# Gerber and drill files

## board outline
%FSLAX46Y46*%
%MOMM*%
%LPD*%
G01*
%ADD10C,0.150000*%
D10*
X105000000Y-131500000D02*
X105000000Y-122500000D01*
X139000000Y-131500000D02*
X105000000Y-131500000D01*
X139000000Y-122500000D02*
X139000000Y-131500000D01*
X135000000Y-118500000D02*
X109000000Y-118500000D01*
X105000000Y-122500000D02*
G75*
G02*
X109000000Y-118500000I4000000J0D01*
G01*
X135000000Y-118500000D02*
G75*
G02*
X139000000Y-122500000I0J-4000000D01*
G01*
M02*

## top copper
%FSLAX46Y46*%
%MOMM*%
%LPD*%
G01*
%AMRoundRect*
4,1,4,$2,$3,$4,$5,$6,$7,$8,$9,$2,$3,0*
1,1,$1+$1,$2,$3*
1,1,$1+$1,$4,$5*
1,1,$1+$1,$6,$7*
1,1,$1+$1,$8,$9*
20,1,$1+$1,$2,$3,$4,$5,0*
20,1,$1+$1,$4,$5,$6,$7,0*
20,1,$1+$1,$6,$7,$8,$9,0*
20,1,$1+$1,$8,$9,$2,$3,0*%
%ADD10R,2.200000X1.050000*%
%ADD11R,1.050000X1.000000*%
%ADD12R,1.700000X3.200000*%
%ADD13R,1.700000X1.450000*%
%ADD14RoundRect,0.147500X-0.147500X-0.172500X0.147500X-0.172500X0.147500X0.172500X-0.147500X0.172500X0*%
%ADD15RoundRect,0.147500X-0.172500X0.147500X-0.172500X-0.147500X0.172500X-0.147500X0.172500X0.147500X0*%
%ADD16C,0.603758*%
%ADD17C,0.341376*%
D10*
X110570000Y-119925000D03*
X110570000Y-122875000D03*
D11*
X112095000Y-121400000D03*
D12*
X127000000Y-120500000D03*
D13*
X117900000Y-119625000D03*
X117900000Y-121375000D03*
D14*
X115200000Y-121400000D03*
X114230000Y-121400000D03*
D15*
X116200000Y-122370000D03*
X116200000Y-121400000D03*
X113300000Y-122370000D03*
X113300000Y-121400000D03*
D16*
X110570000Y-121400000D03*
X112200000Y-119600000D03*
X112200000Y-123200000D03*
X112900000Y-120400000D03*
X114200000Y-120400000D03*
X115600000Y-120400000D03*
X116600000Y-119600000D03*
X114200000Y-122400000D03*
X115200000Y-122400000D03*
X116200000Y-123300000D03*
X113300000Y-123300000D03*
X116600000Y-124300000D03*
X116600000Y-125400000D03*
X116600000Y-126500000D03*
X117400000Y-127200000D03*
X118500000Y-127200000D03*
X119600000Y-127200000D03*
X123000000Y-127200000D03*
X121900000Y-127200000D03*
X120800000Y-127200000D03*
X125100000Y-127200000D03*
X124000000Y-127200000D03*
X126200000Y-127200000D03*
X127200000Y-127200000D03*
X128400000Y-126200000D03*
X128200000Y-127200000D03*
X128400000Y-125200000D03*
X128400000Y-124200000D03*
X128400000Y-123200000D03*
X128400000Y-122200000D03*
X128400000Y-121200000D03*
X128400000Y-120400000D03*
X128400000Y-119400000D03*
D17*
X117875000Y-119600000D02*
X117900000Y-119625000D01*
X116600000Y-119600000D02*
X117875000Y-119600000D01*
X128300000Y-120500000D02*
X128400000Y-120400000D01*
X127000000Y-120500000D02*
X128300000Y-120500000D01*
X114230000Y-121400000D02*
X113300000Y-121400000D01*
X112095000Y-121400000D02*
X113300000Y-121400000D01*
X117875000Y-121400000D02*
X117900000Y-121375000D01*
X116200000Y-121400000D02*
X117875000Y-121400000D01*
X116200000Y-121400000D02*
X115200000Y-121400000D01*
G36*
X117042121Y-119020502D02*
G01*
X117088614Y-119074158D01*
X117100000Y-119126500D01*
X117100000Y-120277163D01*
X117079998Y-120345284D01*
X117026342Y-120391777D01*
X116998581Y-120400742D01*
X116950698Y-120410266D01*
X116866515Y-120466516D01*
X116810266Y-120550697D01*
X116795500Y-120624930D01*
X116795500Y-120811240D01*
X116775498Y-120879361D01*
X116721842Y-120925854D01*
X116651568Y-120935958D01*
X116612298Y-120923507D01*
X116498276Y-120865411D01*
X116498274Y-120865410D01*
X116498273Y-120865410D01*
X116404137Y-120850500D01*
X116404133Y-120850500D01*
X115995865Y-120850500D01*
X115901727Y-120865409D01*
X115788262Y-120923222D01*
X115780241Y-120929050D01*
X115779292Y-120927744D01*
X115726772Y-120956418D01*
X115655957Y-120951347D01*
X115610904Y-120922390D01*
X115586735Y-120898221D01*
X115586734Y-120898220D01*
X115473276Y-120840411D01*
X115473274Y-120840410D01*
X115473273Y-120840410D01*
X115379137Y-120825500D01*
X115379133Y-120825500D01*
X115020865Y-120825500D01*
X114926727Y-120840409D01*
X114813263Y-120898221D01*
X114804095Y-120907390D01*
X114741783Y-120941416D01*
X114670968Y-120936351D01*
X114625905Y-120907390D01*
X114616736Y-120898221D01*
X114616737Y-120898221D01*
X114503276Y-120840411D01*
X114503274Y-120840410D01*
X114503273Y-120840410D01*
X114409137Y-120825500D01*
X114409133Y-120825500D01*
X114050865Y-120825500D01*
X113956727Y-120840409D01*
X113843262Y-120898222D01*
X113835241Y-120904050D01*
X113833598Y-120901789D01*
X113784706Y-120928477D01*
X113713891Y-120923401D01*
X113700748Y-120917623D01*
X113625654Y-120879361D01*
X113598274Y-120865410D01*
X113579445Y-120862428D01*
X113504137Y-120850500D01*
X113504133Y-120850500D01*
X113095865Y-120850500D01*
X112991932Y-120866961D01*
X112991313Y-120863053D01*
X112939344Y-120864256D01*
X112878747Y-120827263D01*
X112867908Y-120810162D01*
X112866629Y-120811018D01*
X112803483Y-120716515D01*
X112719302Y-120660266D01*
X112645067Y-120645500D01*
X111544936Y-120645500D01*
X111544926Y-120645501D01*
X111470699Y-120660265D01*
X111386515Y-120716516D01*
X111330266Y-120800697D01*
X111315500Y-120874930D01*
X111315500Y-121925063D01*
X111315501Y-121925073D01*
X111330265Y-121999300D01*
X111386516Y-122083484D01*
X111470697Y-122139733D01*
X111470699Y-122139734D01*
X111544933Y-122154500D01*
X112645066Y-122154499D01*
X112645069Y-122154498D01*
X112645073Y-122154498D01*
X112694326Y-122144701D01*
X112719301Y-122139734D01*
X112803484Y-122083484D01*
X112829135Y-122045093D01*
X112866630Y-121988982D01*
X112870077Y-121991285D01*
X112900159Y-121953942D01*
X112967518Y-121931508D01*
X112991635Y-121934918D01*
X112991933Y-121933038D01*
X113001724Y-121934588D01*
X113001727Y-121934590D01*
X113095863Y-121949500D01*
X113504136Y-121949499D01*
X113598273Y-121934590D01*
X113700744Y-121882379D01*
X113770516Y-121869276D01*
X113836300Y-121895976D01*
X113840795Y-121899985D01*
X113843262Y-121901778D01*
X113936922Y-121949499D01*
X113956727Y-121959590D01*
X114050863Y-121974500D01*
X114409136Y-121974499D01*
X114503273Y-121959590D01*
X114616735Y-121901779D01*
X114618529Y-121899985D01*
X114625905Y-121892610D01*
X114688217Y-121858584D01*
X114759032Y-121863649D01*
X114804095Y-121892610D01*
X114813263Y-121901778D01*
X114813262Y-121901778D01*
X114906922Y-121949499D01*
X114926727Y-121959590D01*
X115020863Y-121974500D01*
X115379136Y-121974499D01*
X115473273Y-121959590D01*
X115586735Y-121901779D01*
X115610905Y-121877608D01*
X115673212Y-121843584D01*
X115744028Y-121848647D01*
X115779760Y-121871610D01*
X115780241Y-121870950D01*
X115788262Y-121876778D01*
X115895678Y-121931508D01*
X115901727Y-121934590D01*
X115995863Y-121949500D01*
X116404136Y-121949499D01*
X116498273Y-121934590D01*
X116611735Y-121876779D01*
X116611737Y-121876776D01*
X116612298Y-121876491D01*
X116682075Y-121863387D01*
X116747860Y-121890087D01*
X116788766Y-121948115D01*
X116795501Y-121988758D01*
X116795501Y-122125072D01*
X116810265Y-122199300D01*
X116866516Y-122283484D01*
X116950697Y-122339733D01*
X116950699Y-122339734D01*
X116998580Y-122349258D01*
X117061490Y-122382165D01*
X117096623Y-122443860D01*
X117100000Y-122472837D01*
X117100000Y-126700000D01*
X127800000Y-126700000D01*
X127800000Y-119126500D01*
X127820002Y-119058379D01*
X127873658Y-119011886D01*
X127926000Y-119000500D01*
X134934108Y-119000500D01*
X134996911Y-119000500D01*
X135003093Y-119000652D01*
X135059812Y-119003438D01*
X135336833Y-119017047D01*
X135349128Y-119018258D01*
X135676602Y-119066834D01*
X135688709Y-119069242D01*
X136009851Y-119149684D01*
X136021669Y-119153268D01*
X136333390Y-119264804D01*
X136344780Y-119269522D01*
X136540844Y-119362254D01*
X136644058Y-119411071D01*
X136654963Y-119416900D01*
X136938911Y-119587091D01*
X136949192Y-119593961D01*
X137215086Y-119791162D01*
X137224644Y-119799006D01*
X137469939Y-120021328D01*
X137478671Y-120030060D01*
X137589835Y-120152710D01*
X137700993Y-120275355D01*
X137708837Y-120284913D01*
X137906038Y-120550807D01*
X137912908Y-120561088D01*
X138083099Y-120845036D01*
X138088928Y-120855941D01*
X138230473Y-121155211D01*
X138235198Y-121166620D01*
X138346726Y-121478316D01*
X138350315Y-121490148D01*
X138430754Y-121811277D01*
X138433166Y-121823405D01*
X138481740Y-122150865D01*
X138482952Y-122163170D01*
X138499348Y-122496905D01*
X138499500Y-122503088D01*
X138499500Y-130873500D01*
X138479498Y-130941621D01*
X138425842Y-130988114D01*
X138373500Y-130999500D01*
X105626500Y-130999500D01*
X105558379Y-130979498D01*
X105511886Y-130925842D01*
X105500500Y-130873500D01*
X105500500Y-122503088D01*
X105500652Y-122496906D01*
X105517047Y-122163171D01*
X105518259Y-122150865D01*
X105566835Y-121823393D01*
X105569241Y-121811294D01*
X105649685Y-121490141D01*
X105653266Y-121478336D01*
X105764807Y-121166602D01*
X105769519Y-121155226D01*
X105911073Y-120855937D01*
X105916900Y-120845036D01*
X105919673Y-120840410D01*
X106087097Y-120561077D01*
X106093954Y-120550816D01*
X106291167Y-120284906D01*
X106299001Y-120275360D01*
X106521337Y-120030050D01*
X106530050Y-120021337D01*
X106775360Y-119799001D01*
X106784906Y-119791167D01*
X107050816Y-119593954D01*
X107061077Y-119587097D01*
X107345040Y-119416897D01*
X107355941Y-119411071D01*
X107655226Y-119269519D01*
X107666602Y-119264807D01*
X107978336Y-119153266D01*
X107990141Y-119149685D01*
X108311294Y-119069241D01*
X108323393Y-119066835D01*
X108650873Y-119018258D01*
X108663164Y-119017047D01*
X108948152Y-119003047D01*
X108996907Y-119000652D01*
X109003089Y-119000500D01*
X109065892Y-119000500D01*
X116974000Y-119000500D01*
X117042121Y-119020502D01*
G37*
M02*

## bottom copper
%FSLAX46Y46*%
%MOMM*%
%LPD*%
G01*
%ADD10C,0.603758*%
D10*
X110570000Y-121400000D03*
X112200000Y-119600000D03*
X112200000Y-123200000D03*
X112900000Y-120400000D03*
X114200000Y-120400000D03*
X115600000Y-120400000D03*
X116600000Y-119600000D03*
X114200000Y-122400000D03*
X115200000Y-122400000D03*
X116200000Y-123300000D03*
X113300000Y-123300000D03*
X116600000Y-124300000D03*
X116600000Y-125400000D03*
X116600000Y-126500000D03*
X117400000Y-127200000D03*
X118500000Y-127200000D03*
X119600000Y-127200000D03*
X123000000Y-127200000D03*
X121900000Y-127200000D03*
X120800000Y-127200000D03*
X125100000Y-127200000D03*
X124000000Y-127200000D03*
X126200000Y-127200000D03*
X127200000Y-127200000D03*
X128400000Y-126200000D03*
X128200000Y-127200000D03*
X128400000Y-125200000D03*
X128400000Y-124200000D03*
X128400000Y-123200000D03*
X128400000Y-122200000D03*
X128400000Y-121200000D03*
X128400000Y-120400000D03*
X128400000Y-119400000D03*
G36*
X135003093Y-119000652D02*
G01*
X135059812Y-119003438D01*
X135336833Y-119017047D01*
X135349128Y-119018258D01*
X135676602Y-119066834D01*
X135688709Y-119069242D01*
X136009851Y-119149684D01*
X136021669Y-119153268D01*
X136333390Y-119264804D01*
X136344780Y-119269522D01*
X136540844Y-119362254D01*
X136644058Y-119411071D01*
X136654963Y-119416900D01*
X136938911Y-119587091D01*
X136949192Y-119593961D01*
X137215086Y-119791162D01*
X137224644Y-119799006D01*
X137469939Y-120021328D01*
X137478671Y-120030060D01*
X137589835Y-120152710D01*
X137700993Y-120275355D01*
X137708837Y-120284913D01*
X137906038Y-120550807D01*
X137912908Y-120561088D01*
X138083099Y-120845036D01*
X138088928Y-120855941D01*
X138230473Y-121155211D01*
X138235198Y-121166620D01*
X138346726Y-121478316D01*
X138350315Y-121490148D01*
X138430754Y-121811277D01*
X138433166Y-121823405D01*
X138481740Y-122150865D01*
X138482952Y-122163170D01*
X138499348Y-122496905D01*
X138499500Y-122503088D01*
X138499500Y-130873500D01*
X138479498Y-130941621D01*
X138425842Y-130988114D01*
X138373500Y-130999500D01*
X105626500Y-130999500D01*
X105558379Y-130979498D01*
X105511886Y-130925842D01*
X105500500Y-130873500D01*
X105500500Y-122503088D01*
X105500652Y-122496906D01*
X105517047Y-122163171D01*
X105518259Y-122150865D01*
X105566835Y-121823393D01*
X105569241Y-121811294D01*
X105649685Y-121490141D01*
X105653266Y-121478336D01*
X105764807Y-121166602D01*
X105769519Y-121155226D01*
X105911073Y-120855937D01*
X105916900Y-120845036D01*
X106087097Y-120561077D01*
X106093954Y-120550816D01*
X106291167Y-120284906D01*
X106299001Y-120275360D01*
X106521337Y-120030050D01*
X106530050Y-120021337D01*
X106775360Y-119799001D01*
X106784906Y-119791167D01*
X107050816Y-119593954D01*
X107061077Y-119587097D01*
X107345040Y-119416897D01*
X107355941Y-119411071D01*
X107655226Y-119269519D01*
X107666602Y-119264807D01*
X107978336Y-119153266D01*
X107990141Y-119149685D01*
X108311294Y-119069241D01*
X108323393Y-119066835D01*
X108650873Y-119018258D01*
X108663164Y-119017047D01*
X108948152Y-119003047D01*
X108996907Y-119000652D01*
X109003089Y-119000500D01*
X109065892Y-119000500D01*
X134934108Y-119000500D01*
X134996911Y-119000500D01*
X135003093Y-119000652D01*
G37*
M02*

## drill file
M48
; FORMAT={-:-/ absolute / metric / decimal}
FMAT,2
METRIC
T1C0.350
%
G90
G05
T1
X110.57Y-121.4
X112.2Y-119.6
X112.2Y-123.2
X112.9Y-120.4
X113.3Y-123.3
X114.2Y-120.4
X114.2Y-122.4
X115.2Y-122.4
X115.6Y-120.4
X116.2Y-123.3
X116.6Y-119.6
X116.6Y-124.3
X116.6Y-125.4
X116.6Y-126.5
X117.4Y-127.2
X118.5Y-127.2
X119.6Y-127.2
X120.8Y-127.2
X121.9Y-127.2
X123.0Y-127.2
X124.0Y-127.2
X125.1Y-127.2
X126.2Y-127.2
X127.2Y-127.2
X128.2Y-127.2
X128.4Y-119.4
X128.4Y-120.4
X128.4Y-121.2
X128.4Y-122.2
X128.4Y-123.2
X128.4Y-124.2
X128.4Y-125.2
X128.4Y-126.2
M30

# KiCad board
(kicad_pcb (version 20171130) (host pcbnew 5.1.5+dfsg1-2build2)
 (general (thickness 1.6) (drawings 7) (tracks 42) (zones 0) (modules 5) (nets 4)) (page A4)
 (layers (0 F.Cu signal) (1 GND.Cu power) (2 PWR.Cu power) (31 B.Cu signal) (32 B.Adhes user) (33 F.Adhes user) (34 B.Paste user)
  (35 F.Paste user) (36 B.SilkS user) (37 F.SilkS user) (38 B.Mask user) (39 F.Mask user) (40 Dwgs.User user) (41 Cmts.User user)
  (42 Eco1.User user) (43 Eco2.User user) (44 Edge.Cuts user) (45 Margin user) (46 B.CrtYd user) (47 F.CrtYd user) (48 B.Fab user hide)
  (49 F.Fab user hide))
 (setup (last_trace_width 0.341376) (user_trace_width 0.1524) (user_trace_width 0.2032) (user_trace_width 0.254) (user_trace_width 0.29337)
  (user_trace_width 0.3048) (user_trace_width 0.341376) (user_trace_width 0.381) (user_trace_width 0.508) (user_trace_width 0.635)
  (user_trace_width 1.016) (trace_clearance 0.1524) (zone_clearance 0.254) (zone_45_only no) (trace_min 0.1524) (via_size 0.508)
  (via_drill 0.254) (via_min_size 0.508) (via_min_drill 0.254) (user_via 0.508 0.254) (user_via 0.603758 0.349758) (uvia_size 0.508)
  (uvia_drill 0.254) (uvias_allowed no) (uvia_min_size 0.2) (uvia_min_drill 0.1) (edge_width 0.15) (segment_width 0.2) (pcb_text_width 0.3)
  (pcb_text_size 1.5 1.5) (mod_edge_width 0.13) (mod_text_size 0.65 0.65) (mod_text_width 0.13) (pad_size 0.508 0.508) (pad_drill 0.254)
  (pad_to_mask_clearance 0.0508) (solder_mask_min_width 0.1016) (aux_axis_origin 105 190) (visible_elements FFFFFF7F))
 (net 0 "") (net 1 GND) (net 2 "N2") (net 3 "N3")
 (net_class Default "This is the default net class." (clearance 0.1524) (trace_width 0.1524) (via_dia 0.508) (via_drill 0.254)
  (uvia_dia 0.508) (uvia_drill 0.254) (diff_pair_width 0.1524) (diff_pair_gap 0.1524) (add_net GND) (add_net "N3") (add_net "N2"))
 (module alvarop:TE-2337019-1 (layer F.Cu) (at 110.57 121.4 90)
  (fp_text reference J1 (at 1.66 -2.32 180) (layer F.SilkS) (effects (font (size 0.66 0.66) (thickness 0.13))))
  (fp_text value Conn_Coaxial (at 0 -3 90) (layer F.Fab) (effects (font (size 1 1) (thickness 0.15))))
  (pad 2 smd rect (at 1.475 0 90) (size 1.05 2.2) (layers F.Cu F.Paste F.Mask) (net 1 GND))
  (pad 2 smd rect (at -1.475 0 90) (size 1.05 2.2) (layers F.Cu F.Paste F.Mask) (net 1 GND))
  (pad 1 smd rect (at 0 1.525 90) (size 1 1.05) (layers F.Cu F.Paste F.Mask) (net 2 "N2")))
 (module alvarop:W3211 (layer F.Cu) (at 122.45 120.5 180)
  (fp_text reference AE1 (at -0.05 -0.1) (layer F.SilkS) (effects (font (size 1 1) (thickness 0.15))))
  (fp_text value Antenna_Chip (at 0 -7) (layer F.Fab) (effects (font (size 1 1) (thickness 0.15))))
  (pad 2 smd rect (at -4.55 0 180) (size 1.7 3.2) (layers F.Cu F.Paste F.Mask) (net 1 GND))
  (pad 2 smd rect (at 4.55 0.875 180) (size 1.7 1.45) (layers F.Cu F.Paste F.Mask) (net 1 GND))
  (pad 1 smd rect (at 4.55 -0.875 180) (size 1.7 1.45) (layers F.Cu F.Paste F.Mask) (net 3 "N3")))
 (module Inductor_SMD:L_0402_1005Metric (layer F.Cu) (at 114.715 121.4)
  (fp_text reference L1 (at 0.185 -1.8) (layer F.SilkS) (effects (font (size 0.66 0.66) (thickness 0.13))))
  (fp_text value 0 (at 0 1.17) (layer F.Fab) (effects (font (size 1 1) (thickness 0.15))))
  (pad 2 smd roundrect (at 0.485 0) (size 0.59 0.64) (layers F.Cu F.Paste F.Mask) (roundrect_rratio 0.25) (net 3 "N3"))
  (pad 1 smd roundrect (at -0.485 0) (size 0.59 0.64) (layers F.Cu F.Paste F.Mask) (roundrect_rratio 0.25) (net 2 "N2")))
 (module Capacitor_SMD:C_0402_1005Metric (layer F.Cu) (at 116.2 121.885 270)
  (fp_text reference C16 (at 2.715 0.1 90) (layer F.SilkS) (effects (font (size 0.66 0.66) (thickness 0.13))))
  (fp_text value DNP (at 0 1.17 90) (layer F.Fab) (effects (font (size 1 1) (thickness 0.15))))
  (pad 2 smd roundrect (at 0.485 0 270) (size 0.59 0.64) (layers F.Cu F.Paste F.Mask) (roundrect_rratio 0.25) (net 1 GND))
  (pad 1 smd roundrect (at -0.485 0 270) (size 0.59 0.64) (layers F.Cu F.Paste F.Mask) (roundrect_rratio 0.25) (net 3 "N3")))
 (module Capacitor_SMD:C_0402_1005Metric (layer F.Cu) (at 113.3 121.885 270)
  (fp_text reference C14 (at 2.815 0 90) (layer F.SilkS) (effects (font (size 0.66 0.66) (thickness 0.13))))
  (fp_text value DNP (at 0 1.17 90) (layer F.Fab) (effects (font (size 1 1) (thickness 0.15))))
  (pad 2 smd roundrect (at 0.485 0 270) (size 0.59 0.64) (layers F.Cu F.Paste F.Mask) (roundrect_rratio 0.25) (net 1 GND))
  (pad 1 smd roundrect (at -0.485 0 270) (size 0.59 0.64) (layers F.Cu F.Paste F.Mask) (roundrect_rratio 0.25) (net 2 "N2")))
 (gr_line (start 105 131.5) (end 105 122.5) (layer Edge.Cuts) (width 0.15))
 (gr_line (start 139 131.5) (end 105 131.5) (layer Edge.Cuts) (width 0.15))
 (gr_line (start 139 122.5) (end 139 131.5) (layer Edge.Cuts) (width 0.15))
 (gr_line (start 135 118.5) (end 109 118.5) (layer Edge.Cuts) (width 0.15))
 (gr_arc (start 109 122.5) (end 109 118.5) (angle -90) (layer Edge.Cuts) (width 0.15))
 (gr_arc (start 135 122.5) (end 139 122.5) (angle -90) (layer Edge.Cuts) (width 0.15))
 (via (at 110.57 121.4) (size 0.603758) (drill 0.349758) (layers F.Cu B.Cu) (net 1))
 (via (at 112.2 119.6) (size 0.603758) (drill 0.349758) (layers F.Cu B.Cu) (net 1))
 (via (at 112.2 123.2) (size 0.603758) (drill 0.349758) (layers F.Cu B.Cu) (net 1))
 (via (at 112.9 120.4) (size 0.603758) (drill 0.349758) (layers F.Cu B.Cu) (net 1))
 (via (at 114.2 120.4) (size 0.603758) (drill 0.349758) (layers F.Cu B.Cu) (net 1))
 (via (at 115.6 120.4) (size 0.603758) (drill 0.349758) (layers F.Cu B.Cu) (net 1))
 (via (at 116.6 119.6) (size 0.603758) (drill 0.349758) (layers F.Cu B.Cu) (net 1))
 (via (at 114.2 122.4) (size 0.603758) (drill 0.349758) (layers F.Cu B.Cu) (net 1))
 (via (at 115.2 122.4) (size 0.603758) (drill 0.349758) (layers F.Cu B.Cu) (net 1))
 (via (at 116.2 123.3) (size 0.603758) (drill 0.349758) (layers F.Cu B.Cu) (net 1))
 (via (at 113.3 123.3) (size 0.603758) (drill 0.349758) (layers F.Cu B.Cu) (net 1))
 (via (at 116.6 124.3) (size 0.603758) (drill 0.349758) (layers F.Cu B.Cu) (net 1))
 (via (at 116.6 125.4) (size 0.603758) (drill 0.349758) (layers F.Cu B.Cu) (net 1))
 (via (at 116.6 126.5) (size 0.603758) (drill 0.349758) (layers F.Cu B.Cu) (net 1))
 (via (at 117.4 127.2) (size 0.603758) (drill 0.349758) (layers F.Cu B.Cu) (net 1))
 (via (at 118.5 127.2) (size 0.603758) (drill 0.349758) (layers F.Cu B.Cu) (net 1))
 (via (at 119.6 127.2) (size 0.603758) (drill 0.349758) (layers F.Cu B.Cu) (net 1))
 (via (at 123 127.2) (size 0.603758) (drill 0.349758) (layers F.Cu B.Cu) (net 1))
 (via (at 121.9 127.2) (size 0.603758) (drill 0.349758) (layers F.Cu B.Cu) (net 1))
 (via (at 120.8 127.2) (size 0.603758) (drill 0.349758) (layers F.Cu B.Cu) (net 1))
 (via (at 125.1 127.2) (size 0.603758) (drill 0.349758) (layers F.Cu B.Cu) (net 1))
 (via (at 124 127.2) (size 0.603758) (drill 0.349758) (layers F.Cu B.Cu) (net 1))
 (via (at 126.2 127.2) (size 0.603758) (drill 0.349758) (layers F.Cu B.Cu) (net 1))
 (via (at 127.2 127.2) (size 0.603758) (drill 0.349758) (layers F.Cu B.Cu) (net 1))
 (via (at 128.4 126.2) (size 0.603758) (drill 0.349758) (layers F.Cu B.Cu) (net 1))
 (via (at 128.2 127.2) (size 0.603758) (drill 0.349758) (layers F.Cu B.Cu) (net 1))
 (via (at 128.4 125.2) (size 0.603758) (drill 0.349758) (layers F.Cu B.Cu) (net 1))
 (via (at 128.4 124.2) (size 0.603758) (drill 0.349758) (layers F.Cu B.Cu) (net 1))
 (via (at 128.4 123.2) (size 0.603758) (drill 0.349758) (layers F.Cu B.Cu) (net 1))
 (via (at 128.4 122.2) (size 0.603758) (drill 0.349758) (layers F.Cu B.Cu) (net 1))
 (via (at 128.4 121.2) (size 0.603758) (drill 0.349758) (layers F.Cu B.Cu) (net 1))
 (via (at 128.4 120.4) (size 0.603758) (drill 0.349758) (layers F.Cu B.Cu) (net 1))
 (via (at 128.4 119.4) (size 0.603758) (drill 0.349758) (layers F.Cu B.Cu) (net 1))
 (segment (start 117.875 119.6) (end 117.9 119.625) (width 0.341376) (layer F.Cu) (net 1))
 (segment (start 116.6 119.6) (end 117.875 119.6) (width 0.341376) (layer F.Cu) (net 1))
 (segment (start 128.3 120.5) (end 128.4 120.4) (width 0.341376) (layer F.Cu) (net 1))
 (segment (start 127 120.5) (end 128.3 120.5) (width 0.341376) (layer F.Cu) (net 1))
 (segment (start 114.23 121.4) (end 113.3 121.4) (width 0.341376) (layer F.Cu) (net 2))
 (segment (start 112.095 121.4) (end 113.3 121.4) (width 0.341376) (layer F.Cu) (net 2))
 (segment (start 117.875 121.4) (end 117.9 121.375) (width 0.341376) (layer F.Cu) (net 3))
 (segment (start 116.2 121.4) (end 117.875 121.4) (width 0.341376) (layer F.Cu) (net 3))
 (segment (start 116.2 121.4) (end 115.2 121.4) (width 0.341376) (layer F.Cu) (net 3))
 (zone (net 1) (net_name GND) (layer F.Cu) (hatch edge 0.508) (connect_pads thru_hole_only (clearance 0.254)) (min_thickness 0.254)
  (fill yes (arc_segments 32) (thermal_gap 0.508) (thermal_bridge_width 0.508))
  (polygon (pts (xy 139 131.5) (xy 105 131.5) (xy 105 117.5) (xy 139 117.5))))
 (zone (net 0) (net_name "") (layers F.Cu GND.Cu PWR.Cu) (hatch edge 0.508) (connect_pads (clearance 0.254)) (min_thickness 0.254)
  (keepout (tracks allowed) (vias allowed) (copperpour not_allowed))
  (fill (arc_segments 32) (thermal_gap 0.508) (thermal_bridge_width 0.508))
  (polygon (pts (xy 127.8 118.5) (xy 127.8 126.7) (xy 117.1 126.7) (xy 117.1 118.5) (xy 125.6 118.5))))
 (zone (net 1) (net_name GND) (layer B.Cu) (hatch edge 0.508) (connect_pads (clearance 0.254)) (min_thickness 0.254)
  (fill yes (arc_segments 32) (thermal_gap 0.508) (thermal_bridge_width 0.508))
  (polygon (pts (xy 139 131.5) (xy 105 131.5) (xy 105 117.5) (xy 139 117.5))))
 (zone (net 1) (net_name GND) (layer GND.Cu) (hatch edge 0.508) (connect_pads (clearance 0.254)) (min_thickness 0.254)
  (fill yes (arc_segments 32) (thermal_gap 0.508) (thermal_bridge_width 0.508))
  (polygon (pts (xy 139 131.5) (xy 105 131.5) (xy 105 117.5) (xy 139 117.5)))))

